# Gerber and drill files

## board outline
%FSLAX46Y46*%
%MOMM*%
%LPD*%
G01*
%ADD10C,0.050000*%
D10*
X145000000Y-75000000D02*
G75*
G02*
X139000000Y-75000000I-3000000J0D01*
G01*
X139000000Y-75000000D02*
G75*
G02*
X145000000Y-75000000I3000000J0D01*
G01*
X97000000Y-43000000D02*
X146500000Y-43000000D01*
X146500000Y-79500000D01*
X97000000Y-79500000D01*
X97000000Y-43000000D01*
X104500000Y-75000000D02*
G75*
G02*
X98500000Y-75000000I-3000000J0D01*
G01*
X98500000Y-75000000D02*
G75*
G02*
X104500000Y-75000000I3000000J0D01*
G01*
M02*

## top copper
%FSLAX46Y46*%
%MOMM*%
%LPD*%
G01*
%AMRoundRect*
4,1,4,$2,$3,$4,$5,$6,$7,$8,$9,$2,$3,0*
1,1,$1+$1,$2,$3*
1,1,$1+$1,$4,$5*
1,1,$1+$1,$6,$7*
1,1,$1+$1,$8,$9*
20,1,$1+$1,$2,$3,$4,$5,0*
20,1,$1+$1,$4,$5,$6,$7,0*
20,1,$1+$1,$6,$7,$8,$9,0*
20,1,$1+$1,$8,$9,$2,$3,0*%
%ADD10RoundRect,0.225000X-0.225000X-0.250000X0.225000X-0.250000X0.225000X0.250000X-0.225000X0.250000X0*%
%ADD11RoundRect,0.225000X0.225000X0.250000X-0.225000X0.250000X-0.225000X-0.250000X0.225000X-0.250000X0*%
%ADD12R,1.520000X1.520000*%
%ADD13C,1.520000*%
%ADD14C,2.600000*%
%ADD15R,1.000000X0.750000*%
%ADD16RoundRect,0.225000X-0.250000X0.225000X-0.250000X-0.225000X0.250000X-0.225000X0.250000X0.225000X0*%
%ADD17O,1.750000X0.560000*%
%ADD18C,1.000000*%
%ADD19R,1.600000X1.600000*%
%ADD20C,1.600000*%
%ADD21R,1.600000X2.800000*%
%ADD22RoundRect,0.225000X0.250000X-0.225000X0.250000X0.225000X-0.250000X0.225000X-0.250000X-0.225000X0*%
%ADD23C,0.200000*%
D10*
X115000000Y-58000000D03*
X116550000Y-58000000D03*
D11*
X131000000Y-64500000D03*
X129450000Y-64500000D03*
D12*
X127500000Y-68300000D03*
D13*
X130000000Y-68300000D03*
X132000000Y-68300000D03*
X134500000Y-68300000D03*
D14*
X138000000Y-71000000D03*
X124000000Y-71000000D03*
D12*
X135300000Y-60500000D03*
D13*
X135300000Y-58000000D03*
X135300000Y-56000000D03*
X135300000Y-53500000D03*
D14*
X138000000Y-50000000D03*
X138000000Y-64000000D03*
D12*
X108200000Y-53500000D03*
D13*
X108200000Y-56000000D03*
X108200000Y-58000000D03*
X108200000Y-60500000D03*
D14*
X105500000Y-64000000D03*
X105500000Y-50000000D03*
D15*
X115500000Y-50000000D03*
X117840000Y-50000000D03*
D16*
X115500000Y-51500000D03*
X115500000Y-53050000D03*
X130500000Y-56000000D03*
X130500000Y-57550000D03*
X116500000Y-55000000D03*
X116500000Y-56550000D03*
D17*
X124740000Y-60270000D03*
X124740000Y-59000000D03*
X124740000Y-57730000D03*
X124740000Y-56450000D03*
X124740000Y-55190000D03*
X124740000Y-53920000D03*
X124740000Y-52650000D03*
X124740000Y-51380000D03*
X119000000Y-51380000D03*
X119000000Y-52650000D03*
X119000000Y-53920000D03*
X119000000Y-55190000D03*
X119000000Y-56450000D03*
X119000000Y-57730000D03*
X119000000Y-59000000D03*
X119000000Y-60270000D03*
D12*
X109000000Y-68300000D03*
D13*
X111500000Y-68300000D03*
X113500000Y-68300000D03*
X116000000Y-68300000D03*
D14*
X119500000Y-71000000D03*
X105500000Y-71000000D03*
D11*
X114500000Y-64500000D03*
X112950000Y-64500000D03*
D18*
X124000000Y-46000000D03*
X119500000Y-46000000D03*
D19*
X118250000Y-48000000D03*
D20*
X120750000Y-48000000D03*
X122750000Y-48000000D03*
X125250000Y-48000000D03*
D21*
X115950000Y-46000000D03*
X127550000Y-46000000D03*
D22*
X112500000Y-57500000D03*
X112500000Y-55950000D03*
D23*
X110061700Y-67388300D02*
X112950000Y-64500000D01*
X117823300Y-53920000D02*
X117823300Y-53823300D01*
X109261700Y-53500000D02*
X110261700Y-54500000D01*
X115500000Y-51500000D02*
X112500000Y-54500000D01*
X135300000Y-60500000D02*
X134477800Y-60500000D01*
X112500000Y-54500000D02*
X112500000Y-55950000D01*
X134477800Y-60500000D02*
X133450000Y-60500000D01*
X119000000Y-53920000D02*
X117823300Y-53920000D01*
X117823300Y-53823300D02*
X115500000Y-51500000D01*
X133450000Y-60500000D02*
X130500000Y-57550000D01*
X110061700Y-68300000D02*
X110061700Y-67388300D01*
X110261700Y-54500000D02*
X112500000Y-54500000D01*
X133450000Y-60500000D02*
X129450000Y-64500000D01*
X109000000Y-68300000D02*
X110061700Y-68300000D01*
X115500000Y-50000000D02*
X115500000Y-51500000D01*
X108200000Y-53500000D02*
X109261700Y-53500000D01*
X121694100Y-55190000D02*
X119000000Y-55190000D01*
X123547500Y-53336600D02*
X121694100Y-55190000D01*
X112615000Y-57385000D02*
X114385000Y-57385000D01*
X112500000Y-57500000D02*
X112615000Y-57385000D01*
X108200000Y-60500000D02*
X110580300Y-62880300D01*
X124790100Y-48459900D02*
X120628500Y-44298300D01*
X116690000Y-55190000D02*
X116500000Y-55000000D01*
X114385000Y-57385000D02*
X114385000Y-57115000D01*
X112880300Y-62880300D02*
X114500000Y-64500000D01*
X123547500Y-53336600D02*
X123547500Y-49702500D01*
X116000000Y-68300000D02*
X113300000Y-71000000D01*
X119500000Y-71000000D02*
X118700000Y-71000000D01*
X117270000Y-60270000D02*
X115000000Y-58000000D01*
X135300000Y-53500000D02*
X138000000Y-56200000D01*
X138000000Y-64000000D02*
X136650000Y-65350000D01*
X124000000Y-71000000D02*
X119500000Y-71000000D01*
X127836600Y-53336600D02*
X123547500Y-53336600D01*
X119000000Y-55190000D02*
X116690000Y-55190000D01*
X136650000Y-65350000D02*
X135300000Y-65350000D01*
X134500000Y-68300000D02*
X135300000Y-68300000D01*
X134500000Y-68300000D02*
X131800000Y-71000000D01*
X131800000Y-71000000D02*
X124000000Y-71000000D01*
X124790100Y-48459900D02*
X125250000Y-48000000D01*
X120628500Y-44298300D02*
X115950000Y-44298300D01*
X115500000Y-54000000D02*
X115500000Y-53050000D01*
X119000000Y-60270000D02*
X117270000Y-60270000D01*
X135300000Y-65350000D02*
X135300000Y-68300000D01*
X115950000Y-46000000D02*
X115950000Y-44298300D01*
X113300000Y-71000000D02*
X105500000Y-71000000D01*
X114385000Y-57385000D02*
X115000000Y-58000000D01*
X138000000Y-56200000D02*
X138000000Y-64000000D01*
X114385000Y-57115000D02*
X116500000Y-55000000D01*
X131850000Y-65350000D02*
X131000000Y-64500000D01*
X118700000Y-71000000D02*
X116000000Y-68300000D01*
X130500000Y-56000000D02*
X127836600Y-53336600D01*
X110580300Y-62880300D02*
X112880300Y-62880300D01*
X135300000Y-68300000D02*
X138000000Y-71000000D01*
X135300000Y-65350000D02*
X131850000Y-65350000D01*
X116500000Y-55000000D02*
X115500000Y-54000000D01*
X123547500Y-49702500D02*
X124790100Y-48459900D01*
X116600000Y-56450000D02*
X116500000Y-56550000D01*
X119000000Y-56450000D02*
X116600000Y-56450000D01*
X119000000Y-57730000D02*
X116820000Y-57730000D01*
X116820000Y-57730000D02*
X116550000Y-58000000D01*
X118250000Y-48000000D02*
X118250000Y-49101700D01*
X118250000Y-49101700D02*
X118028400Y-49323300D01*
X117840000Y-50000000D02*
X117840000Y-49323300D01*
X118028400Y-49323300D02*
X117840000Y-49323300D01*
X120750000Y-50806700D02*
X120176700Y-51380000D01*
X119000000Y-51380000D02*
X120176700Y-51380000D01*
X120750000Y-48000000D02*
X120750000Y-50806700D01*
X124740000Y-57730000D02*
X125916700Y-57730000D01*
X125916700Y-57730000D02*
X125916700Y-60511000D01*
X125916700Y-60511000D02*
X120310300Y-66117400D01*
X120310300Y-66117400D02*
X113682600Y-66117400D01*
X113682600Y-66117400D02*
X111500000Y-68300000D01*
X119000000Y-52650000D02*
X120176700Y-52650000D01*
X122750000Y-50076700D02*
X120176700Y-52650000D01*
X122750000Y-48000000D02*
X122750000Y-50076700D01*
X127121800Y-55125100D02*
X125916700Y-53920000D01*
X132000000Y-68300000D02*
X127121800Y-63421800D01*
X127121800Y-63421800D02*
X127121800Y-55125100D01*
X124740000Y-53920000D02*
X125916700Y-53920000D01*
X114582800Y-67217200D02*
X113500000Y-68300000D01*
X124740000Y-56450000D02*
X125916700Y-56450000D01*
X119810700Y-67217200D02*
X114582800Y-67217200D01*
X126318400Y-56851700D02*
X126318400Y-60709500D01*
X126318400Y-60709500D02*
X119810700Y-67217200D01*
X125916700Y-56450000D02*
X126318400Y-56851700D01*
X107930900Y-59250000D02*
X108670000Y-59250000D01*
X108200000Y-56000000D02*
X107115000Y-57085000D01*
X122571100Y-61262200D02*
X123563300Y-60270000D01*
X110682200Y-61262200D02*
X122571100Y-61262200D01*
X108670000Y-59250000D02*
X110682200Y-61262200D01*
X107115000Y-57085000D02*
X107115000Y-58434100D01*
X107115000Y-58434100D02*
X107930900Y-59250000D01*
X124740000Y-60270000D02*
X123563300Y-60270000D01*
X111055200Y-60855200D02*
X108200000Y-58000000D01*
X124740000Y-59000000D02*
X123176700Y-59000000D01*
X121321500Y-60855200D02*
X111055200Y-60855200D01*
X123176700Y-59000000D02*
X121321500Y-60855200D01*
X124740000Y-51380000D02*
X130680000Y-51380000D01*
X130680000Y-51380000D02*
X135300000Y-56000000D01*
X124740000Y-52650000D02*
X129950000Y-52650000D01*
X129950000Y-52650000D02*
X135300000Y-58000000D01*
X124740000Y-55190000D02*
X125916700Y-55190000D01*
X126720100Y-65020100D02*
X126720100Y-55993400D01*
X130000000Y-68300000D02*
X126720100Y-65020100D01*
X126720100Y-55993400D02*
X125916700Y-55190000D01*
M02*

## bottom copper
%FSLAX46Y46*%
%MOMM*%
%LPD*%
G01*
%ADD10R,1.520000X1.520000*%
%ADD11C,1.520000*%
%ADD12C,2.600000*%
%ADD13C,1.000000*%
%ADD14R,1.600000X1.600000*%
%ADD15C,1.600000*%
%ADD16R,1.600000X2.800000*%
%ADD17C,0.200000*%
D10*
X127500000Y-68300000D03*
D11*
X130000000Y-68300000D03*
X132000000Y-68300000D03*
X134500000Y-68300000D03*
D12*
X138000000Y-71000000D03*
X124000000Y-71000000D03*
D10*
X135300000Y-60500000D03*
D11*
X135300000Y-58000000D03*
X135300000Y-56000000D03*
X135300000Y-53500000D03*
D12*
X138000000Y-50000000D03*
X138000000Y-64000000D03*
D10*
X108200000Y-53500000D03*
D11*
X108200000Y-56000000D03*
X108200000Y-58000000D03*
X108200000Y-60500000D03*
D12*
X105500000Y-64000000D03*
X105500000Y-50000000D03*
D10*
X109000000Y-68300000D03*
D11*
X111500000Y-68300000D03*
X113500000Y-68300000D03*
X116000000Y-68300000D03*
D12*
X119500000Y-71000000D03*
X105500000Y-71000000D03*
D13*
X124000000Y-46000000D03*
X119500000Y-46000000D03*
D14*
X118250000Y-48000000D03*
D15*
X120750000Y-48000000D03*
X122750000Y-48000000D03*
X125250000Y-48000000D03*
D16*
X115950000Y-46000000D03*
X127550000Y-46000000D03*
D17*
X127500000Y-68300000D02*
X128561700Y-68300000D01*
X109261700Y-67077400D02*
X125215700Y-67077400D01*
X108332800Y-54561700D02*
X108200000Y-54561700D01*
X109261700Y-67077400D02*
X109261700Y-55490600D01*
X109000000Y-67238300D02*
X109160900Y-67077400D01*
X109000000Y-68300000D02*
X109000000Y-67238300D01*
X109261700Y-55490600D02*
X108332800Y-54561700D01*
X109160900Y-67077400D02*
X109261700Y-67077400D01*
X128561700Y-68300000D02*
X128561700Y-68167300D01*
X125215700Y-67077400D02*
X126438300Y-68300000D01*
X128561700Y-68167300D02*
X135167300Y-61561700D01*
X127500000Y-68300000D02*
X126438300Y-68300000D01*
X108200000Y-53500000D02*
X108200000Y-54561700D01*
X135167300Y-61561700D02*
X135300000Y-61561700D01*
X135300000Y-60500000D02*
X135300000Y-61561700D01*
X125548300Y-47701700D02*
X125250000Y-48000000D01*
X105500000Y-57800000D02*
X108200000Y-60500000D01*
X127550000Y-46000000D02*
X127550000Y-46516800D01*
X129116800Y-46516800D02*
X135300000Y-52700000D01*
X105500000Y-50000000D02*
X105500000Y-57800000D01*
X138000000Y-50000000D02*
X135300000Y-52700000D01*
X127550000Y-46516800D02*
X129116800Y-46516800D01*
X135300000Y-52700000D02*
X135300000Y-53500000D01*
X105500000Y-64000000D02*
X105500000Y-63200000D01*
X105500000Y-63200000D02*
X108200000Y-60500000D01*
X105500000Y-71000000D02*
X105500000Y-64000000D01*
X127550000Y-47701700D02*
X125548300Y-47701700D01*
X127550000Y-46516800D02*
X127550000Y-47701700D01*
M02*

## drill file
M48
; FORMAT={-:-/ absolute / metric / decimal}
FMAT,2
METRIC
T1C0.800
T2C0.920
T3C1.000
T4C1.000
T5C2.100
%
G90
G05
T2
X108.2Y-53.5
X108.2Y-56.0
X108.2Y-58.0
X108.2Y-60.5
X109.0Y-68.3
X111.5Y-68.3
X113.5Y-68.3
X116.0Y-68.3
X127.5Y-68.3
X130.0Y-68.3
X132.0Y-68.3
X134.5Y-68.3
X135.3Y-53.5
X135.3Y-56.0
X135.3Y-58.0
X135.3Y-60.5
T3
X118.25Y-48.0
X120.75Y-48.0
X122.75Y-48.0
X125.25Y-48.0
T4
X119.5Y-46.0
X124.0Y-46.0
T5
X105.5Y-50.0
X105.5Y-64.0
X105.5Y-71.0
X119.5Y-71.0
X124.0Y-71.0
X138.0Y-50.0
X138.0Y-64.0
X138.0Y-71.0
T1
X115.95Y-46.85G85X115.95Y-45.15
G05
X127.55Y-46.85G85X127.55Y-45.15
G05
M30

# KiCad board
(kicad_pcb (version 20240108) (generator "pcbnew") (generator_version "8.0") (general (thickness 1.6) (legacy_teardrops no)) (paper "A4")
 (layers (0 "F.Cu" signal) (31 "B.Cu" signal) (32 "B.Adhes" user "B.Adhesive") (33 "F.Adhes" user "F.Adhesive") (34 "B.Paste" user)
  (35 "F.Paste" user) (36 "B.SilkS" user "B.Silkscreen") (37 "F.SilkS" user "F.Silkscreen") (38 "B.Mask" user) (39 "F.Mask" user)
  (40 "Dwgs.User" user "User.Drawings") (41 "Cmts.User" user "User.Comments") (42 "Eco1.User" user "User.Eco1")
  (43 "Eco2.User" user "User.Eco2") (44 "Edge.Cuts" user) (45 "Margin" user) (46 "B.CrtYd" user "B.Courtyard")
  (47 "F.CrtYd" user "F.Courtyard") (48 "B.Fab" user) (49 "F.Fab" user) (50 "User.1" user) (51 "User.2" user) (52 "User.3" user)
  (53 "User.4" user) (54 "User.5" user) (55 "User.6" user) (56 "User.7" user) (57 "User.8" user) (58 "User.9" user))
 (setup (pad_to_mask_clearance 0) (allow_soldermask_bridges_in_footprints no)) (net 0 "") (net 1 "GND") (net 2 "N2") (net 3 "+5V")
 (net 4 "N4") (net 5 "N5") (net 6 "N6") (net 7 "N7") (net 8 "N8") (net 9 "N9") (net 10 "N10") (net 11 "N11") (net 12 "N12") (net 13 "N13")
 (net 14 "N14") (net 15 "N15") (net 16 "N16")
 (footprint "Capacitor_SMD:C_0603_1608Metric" (layer "F.Cu") (at 115.775 58)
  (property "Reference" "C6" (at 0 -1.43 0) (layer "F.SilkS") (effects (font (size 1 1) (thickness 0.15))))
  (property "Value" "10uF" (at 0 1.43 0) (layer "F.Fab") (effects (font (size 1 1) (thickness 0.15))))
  (pad "1" smd roundrect (at -0.775 0) (size 0.9 0.95) (layers "F.Cu" "F.Paste" "F.Mask") (roundrect_rratio 0.25) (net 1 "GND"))
  (pad "2" smd roundrect (at 0.775 0) (size 0.9 0.95) (layers "F.Cu" "F.Paste" "F.Mask") (roundrect_rratio 0.25) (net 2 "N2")))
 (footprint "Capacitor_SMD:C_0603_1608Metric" (layer "F.Cu") (at 130.225 64.5 180)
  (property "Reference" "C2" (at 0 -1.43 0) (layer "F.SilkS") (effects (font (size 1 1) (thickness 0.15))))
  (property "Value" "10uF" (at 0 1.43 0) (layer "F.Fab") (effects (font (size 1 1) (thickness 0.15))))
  (pad "1" smd roundrect (at -0.775 0 180) (size 0.9 0.95) (layers "F.Cu" "F.Paste" "F.Mask") (roundrect_rratio 0.25) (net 1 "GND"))
  (pad "2" smd roundrect (at 0.775 0 180) (size 0.9 0.95) (layers "F.Cu" "F.Paste" "F.Mask") (roundrect_rratio 0.25) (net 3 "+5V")))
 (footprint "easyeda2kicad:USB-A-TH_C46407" (layer "F.Cu") (at 131 69.65)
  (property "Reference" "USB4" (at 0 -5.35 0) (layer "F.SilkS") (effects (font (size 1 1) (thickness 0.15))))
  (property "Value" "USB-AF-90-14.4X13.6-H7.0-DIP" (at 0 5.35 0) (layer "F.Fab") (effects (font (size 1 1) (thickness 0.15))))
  (pad "1" thru_hole rect (at -3.5 -1.35) (size 1.52 1.52) (drill 0.919988) (layers "*.Cu" "*.Mask") (remove_unused_layers no) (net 3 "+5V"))
  (pad "2" thru_hole circle (at -1 -1.35) (size 1.52 1.52) (drill 0.919988) (layers "*.Cu" "*.Mask") (remove_unused_layers no) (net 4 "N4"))
  (pad "3" thru_hole circle (at 1 -1.35) (size 1.52 1.52) (drill 0.919988) (layers "*.Cu" "*.Mask") (remove_unused_layers no) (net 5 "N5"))
  (pad "4" thru_hole circle (at 3.5 -1.35) (size 1.52 1.52) (drill 0.919988) (layers "*.Cu" "*.Mask") (remove_unused_layers no)
   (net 1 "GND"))
  (pad "5" thru_hole circle (at 7 1.35) (size 2.6 2.6) (drill 2.100021) (layers "*.Cu" "*.Mask") (remove_unused_layers no) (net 1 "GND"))
  (pad "6" thru_hole circle (at -7 1.35) (size 2.6 2.6) (drill 2.100021) (layers "*.Cu" "*.Mask") (remove_unused_layers no) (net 1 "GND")))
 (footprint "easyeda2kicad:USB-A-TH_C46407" (layer "F.Cu") (at 136.65 57 90)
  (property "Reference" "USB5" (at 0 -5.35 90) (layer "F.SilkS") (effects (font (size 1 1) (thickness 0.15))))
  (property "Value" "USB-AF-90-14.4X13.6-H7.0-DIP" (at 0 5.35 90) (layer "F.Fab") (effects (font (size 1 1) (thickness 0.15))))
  (pad "1" thru_hole rect (at -3.5 -1.35 90) (size 1.52 1.52) (drill 0.919988) (layers "*.Cu" "*.Mask") (remove_unused_layers no)
   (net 3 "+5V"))
  (pad "2" thru_hole circle (at -1 -1.35 90) (size 1.52 1.52) (drill 0.919988) (layers "*.Cu" "*.Mask") (remove_unused_layers no)
   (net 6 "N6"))
  (pad "3" thru_hole circle (at 1 -1.35 90) (size 1.52 1.52) (drill 0.919988) (layers "*.Cu" "*.Mask") (remove_unused_layers no)
   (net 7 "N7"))
  (pad "4" thru_hole circle (at 3.5 -1.35 90) (size 1.52 1.52) (drill 0.919988) (layers "*.Cu" "*.Mask") (remove_unused_layers no)
   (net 1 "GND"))
  (pad "5" thru_hole circle (at 7 1.35 90) (size 2.6 2.6) (drill 2.100021) (layers "*.Cu" "*.Mask") (remove_unused_layers no) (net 1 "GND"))
  (pad "6" thru_hole circle (at -7 1.35 90) (size 2.6 2.6) (drill 2.100021) (layers "*.Cu" "*.Mask") (remove_unused_layers no) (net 1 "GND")))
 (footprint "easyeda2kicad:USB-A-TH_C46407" (layer "F.Cu") (at 106.85 57 -90)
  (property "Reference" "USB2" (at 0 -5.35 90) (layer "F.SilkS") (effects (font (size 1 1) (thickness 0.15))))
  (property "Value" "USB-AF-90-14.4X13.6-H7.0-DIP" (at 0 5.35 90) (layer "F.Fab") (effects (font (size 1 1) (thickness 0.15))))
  (pad "1" thru_hole rect (at -3.5 -1.35 270) (size 1.52 1.52) (drill 0.919988) (layers "*.Cu" "*.Mask") (remove_unused_layers no)
   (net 3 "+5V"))
  (pad "2" thru_hole circle (at -1 -1.35 270) (size 1.52 1.52) (drill 0.919988) (layers "*.Cu" "*.Mask") (remove_unused_layers no)
   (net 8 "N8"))
  (pad "3" thru_hole circle (at 1 -1.35 270) (size 1.52 1.52) (drill 0.919988) (layers "*.Cu" "*.Mask") (remove_unused_layers no)
   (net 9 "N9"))
  (pad "4" thru_hole circle (at 3.5 -1.35 270) (size 1.52 1.52) (drill 0.919988) (layers "*.Cu" "*.Mask") (remove_unused_layers no)
   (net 1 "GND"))
  (pad "5" thru_hole circle (at 7 1.35 270) (size 2.6 2.6) (drill 2.100021) (layers "*.Cu" "*.Mask") (remove_unused_layers no) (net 1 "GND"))
  (pad "6" thru_hole circle (at -7 1.35 270) (size 2.6 2.6) (drill 2.100021) (layers "*.Cu" "*.Mask") (remove_unused_layers no)
   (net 1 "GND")))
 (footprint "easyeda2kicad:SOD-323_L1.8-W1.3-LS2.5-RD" (layer "F.Cu") (at 116.67 50)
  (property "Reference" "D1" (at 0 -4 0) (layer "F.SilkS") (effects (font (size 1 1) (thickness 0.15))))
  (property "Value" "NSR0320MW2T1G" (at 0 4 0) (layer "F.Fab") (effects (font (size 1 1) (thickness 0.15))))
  (pad "1" smd rect (at -1.17 0) (size 1 0.75) (layers "F.Cu" "F.Paste" "F.Mask") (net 3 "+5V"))
  (pad "2" smd rect (at 1.17 0) (size 1 0.75) (layers "F.Cu" "F.Paste" "F.Mask") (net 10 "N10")))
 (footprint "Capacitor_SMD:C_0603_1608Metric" (layer "F.Cu") (at 115.5 52.275 -90)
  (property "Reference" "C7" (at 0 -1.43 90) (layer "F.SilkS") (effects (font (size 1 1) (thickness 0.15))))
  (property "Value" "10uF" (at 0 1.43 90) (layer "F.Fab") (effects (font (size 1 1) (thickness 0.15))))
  (pad "1" smd roundrect (at -0.775 0 270) (size 0.9 0.95) (layers "F.Cu" "F.Paste" "F.Mask") (roundrect_rratio 0.25) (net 3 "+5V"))
  (pad "2" smd roundrect (at 0.775 0 270) (size 0.9 0.95) (layers "F.Cu" "F.Paste" "F.Mask") (roundrect_rratio 0.25) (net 1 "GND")))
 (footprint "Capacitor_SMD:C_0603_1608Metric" (layer "F.Cu") (at 130.5 56.775 -90)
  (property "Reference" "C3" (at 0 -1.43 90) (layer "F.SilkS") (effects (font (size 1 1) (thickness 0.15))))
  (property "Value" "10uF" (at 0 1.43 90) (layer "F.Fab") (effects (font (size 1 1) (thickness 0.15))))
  (pad "1" smd roundrect (at -0.775 0 270) (size 0.9 0.95) (layers "F.Cu" "F.Paste" "F.Mask") (roundrect_rratio 0.25) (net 1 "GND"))
  (pad "2" smd roundrect (at 0.775 0 270) (size 0.9 0.95) (layers "F.Cu" "F.Paste" "F.Mask") (roundrect_rratio 0.25) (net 3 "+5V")))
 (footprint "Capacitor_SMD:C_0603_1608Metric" (layer "F.Cu") (at 116.5 55.775 -90)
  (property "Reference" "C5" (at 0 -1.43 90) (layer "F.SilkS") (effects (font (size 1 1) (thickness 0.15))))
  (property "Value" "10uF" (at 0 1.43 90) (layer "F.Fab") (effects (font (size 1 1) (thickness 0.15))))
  (pad "1" smd roundrect (at -0.775 0 270) (size 0.9 0.95) (layers "F.Cu" "F.Paste" "F.Mask") (roundrect_rratio 0.25) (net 1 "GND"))
  (pad "2" smd roundrect (at 0.775 0 270) (size 0.9 0.95) (layers "F.Cu" "F.Paste" "F.Mask") (roundrect_rratio 0.25) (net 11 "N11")))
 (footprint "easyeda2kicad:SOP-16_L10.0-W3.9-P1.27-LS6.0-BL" (layer "F.Cu") (at 121.87 55.82 90)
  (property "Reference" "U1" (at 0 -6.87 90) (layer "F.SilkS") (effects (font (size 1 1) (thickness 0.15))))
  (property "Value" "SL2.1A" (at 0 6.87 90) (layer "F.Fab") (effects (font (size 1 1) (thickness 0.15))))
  (pad "1" smd oval (at -4.45 2.87 90) (size 0.56 1.75) (layers "F.Cu" "F.Paste" "F.Mask") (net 8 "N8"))
  (pad "2" smd oval (at -3.18 2.87 90) (size 0.56 1.75) (layers "F.Cu" "F.Paste" "F.Mask") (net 9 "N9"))
  (pad "3" smd oval (at -1.91 2.87 90) (size 0.56 1.75) (layers "F.Cu" "F.Paste" "F.Mask") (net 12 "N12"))
  (pad "4" smd oval (at -0.63 2.87 90) (size 0.56 1.75) (layers "F.Cu" "F.Paste" "F.Mask") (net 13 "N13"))
  (pad "5" smd oval (at 0.63 2.87 90) (size 0.56 1.75) (layers "F.Cu" "F.Paste" "F.Mask") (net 4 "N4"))
  (pad "6" smd oval (at 1.9 2.87 90) (size 0.56 1.75) (layers "F.Cu" "F.Paste" "F.Mask") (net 5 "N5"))
  (pad "7" smd oval (at 3.17 2.87 90) (size 0.56 1.75) (layers "F.Cu" "F.Paste" "F.Mask") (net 6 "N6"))
  (pad "8" smd oval (at 4.44 2.87 90) (size 0.56 1.75) (layers "F.Cu" "F.Paste" "F.Mask") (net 7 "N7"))
  (pad "9" smd oval (at 4.44 -2.87 90) (size 0.56 1.75) (layers "F.Cu" "F.Paste" "F.Mask") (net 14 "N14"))
  (pad "10" smd oval (at 3.17 -2.87 90) (size 0.56 1.75) (layers "F.Cu" "F.Paste" "F.Mask") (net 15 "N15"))
  (pad "11" smd oval (at 1.9 -2.87 90) (size 0.56 1.75) (layers "F.Cu" "F.Paste" "F.Mask") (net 3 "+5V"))
  (pad "12" smd oval (at 0.63 -2.87 90) (size 0.56 1.75) (layers "F.Cu" "F.Paste" "F.Mask") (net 1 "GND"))
  (pad "13" smd oval (at -0.63 -2.87 90) (size 0.56 1.75) (layers "F.Cu" "F.Paste" "F.Mask") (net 11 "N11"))
  (pad "14" smd oval (at -1.91 -2.87 90) (size 0.56 1.75) (layers "F.Cu" "F.Paste" "F.Mask") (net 2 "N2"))
  (pad "15" smd oval (at -3.18 -2.87 90) (size 0.56 1.75) (layers "F.Cu" "F.Paste" "F.Mask") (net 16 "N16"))
  (pad "16" smd oval (at -4.45 -2.87 90) (size 0.56 1.75) (layers "F.Cu" "F.Paste" "F.Mask") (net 1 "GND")))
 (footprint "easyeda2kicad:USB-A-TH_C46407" (layer "F.Cu") (at 112.5 69.65)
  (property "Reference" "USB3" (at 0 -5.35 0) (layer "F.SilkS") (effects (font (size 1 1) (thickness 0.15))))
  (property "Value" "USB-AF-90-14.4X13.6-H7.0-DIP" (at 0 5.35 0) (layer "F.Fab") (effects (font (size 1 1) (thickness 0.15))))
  (pad "1" thru_hole rect (at -3.5 -1.35) (size 1.52 1.52) (drill 0.919988) (layers "*.Cu" "*.Mask") (remove_unused_layers no) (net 3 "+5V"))
  (pad "2" thru_hole circle (at -1 -1.35) (size 1.52 1.52) (drill 0.919988) (layers "*.Cu" "*.Mask") (remove_unused_layers no)
   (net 12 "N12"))
  (pad "3" thru_hole circle (at 1 -1.35) (size 1.52 1.52) (drill 0.919988) (layers "*.Cu" "*.Mask") (remove_unused_layers no) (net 13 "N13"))
  (pad "4" thru_hole circle (at 3.5 -1.35) (size 1.52 1.52) (drill 0.919988) (layers "*.Cu" "*.Mask") (remove_unused_layers no)
   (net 1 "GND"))
  (pad "5" thru_hole circle (at 7 1.35) (size 2.6 2.6) (drill 2.100021) (layers "*.Cu" "*.Mask") (remove_unused_layers no) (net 1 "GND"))
  (pad "6" thru_hole circle (at -7 1.35) (size 2.6 2.6) (drill 2.100021) (layers "*.Cu" "*.Mask") (remove_unused_layers no) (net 1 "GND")))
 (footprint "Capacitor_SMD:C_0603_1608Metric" (layer "F.Cu") (at 113.725 64.5 180)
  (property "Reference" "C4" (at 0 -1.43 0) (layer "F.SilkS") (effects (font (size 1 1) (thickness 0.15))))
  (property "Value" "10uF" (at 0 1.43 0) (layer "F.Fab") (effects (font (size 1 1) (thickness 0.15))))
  (pad "1" smd roundrect (at -0.775 0 180) (size 0.9 0.95) (layers "F.Cu" "F.Paste" "F.Mask") (roundrect_rratio 0.25) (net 1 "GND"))
  (pad "2" smd roundrect (at 0.775 0 180) (size 0.9 0.95) (layers "F.Cu" "F.Paste" "F.Mask") (roundrect_rratio 0.25) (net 3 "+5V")))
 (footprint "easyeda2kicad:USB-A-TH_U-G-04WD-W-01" (layer "F.Cu") (at 121.75 47 180)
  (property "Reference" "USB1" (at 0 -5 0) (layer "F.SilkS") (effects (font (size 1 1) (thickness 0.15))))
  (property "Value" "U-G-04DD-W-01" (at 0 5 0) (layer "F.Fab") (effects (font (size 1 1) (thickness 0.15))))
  (pad "" thru_hole circle (at -2.25 1 180) (size 1 1) (drill 1) (layers "*.Cu" "*.Mask") (remove_unused_layers no))
  (pad "" thru_hole circle (at 2.25 1 180) (size 1 1) (drill 1) (layers "*.Cu" "*.Mask") (remove_unused_layers no))
  (pad "1" thru_hole rect (at 3.5 -1 180) (size 1.6 1.6) (drill 0.999998) (layers "*.Cu" "*.Mask") (remove_unused_layers no) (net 10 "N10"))
  (pad "2" thru_hole circle (at 1 -1 180) (size 1.6 1.6) (drill 0.999998) (layers "*.Cu" "*.Mask") (remove_unused_layers no) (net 14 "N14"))
  (pad "3" thru_hole circle (at -1 -1 180) (size 1.6 1.6) (drill 0.999998) (layers "*.Cu" "*.Mask") (remove_unused_layers no) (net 15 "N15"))
  (pad "4" thru_hole circle (at -3.5 -1 180) (size 1.6 1.6) (drill 0.999998) (layers "*.Cu" "*.Mask") (remove_unused_layers no)
   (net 1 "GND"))
  (pad "5" thru_hole rect (at 5.8 1 180) (size 1.6 2.8) (drill oval 0.799998 2.499995) (layers "*.Cu" "*.Mask") (remove_unused_layers no)
   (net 1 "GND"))
  (pad "6" thru_hole rect (at -5.8 1 180) (size 1.6 2.8) (drill oval 0.799998 2.499995) (layers "*.Cu" "*.Mask") (remove_unused_layers no)
   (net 1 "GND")))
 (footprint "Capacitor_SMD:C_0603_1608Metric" (layer "F.Cu") (at 112.5 56.725 90)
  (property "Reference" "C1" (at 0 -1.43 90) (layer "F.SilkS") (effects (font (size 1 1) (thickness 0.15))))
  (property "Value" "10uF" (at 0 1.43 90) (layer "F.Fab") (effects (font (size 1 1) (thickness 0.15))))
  (pad "1" smd roundrect (at -0.775 0 90) (size 0.9 0.95) (layers "F.Cu" "F.Paste" "F.Mask") (roundrect_rratio 0.25) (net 1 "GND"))
  (pad "2" smd roundrect (at 0.775 0 90) (size 0.9 0.95) (layers "F.Cu" "F.Paste" "F.Mask") (roundrect_rratio 0.25) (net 3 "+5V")))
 (gr_circle (center 142 75) (end 145 75) (stroke (width 0.05) (type default)) (fill none) (layer "Edge.Cuts"))
 (gr_rect (start 97 43) (end 146.5 79.5) (stroke (width 0.05) (type default)) (fill none) (layer "Edge.Cuts"))
 (gr_circle (center 101.5 75) (end 104.5 75) (stroke (width 0.05) (type default)) (fill none) (layer "Edge.Cuts"))
 (segment (start 110.0617 67.3883) (end 112.95 64.5) (width 0.2) (layer "F.Cu") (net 3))
 (segment (start 117.8233 53.92) (end 117.8233 53.8233) (width 0.2) (layer "F.Cu") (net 3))
 (segment (start 109.2617 53.5) (end 110.2617 54.5) (width 0.2) (layer "F.Cu") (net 3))
 (segment (start 115.5 51.5) (end 112.5 54.5) (width 0.2) (layer "F.Cu") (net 3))
 (segment (start 135.3 60.5) (end 134.4778 60.5) (width 0.2) (layer "F.Cu") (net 3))
 (segment (start 112.5 54.5) (end 112.5 55.95) (width 0.2) (layer "F.Cu") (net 3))
 (segment (start 134.4778 60.5) (end 133.45 60.5) (width 0.2) (layer "F.Cu") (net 3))
 (segment (start 119 53.92) (end 117.8233 53.92) (width 0.2) (layer "F.Cu") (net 3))
 (segment (start 117.8233 53.8233) (end 115.5 51.5) (width 0.2) (layer "F.Cu") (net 3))
 (segment (start 133.45 60.5) (end 130.5 57.55) (width 0.2) (layer "F.Cu") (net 3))
 (segment (start 110.0617 68.3) (end 110.0617 67.3883) (width 0.2) (layer "F.Cu") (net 3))
 (segment (start 110.2617 54.5) (end 112.5 54.5) (width 0.2) (layer "F.Cu") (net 3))
 (segment (start 133.45 60.5) (end 129.45 64.5) (width 0.2) (layer "F.Cu") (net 3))
 (segment (start 109 68.3) (end 110.0617 68.3) (width 0.2) (layer "F.Cu") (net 3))
 (segment (start 115.5 50) (end 115.5 51.5) (width 0.2) (layer "F.Cu") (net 3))
 (segment (start 108.2 53.5) (end 109.2617 53.5) (width 0.2) (layer "F.Cu") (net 3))
 (segment (start 127.5 68.3) (end 128.5617 68.3) (width 0.2) (layer "B.Cu") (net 3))
 (segment (start 109.2617 67.0774) (end 125.2157 67.0774) (width 0.2) (layer "B.Cu") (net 3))
 (segment (start 108.3328 54.5617) (end 108.2 54.5617) (width 0.2) (layer "B.Cu") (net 3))
 (segment (start 109.2617 67.0774) (end 109.2617 55.4906) (width 0.2) (layer "B.Cu") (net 3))
 (segment (start 109 67.2383) (end 109.1609 67.0774) (width 0.2) (layer "B.Cu") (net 3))
 (segment (start 109 68.3) (end 109 67.2383) (width 0.2) (layer "B.Cu") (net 3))
 (segment (start 109.2617 55.4906) (end 108.3328 54.5617) (width 0.2) (layer "B.Cu") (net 3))
 (segment (start 109.1609 67.0774) (end 109.2617 67.0774) (width 0.2) (layer "B.Cu") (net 3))
 (segment (start 128.5617 68.3) (end 128.5617 68.1673) (width 0.2) (layer "B.Cu") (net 3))
 (segment (start 125.2157 67.0774) (end 126.4383 68.3) (width 0.2) (layer "B.Cu") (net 3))
 (segment (start 128.5617 68.1673) (end 135.1673 61.5617) (width 0.2) (layer "B.Cu") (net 3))
 (segment (start 127.5 68.3) (end 126.4383 68.3) (width 0.2) (layer "B.Cu") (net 3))
 (segment (start 108.2 53.5) (end 108.2 54.5617) (width 0.2) (layer "B.Cu") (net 3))
 (segment (start 135.1673 61.5617) (end 135.3 61.5617) (width 0.2) (layer "B.Cu") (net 3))
 (segment (start 135.3 60.5) (end 135.3 61.5617) (width 0.2) (layer "B.Cu") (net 3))
 (segment (start 121.6941 55.19) (end 119 55.19) (width 0.2) (layer "F.Cu") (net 1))
 (segment (start 123.5475 53.3366) (end 121.6941 55.19) (width 0.2) (layer "F.Cu") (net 1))
 (segment (start 112.615 57.385) (end 114.385 57.385) (width 0.2) (layer "F.Cu") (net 1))
 (segment (start 112.5 57.5) (end 112.615 57.385) (width 0.2) (layer "F.Cu") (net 1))
 (segment (start 108.2 60.5) (end 110.5803 62.8803) (width 0.2) (layer "F.Cu") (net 1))
 (segment (start 124.7901 48.4599) (end 120.6285 44.2983) (width 0.2) (layer "F.Cu") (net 1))
 (segment (start 116.69 55.19) (end 116.5 55) (width 0.2) (layer "F.Cu") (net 1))
 (segment (start 114.385 57.385) (end 114.385 57.115) (width 0.2) (layer "F.Cu") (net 1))
 (segment (start 112.8803 62.8803) (end 114.5 64.5) (width 0.2) (layer "F.Cu") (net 1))
 (segment (start 123.5475 53.3366) (end 123.5475 49.7025) (width 0.2) (layer "F.Cu") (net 1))
 (segment (start 116 68.3) (end 113.3 71) (width 0.2) (layer "F.Cu") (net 1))
 (segment (start 119.5 71) (end 118.7 71) (width 0.2) (layer "F.Cu") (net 1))
 (segment (start 117.27 60.27) (end 115 58) (width 0.2) (layer "F.Cu") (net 1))
 (segment (start 135.3 53.5) (end 138 56.2) (width 0.2) (layer "F.Cu") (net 1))
 (segment (start 138 64) (end 136.65 65.35) (width 0.2) (layer "F.Cu") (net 1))
 (segment (start 124 71) (end 119.5 71) (width 0.2) (layer "F.Cu") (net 1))
 (segment (start 127.8366 53.3366) (end 123.5475 53.3366) (width 0.2) (layer "F.Cu") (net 1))
 (segment (start 119 55.19) (end 116.69 55.19) (width 0.2) (layer "F.Cu") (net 1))
 (segment (start 136.65 65.35) (end 135.3 65.35) (width 0.2) (layer "F.Cu") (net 1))
 (segment (start 134.5 68.3) (end 135.3 68.3) (width 0.2) (layer "F.Cu") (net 1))
 (segment (start 134.5 68.3) (end 131.8 71) (width 0.2) (layer "F.Cu") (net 1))
 (segment (start 131.8 71) (end 124 71) (width 0.2) (layer "F.Cu") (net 1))
 (segment (start 124.7901 48.4599) (end 125.25 48) (width 0.2) (layer "F.Cu") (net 1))
 (segment (start 120.6285 44.2983) (end 115.95 44.2983) (width 0.2) (layer "F.Cu") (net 1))
 (segment (start 115.5 54) (end 115.5 53.05) (width 0.2) (layer "F.Cu") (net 1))
 (segment (start 119 60.27) (end 117.27 60.27) (width 0.2) (layer "F.Cu") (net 1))
 (segment (start 135.3 65.35) (end 135.3 68.3) (width 0.2) (layer "F.Cu") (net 1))
 (segment (start 115.95 46) (end 115.95 44.2983) (width 0.2) (layer "F.Cu") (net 1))
 (segment (start 113.3 71) (end 105.5 71) (width 0.2) (layer "F.Cu") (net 1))
 (segment (start 114.385 57.385) (end 115 58) (width 0.2) (layer "F.Cu") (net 1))
 (segment (start 138 56.2) (end 138 64) (width 0.2) (layer "F.Cu") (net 1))
 (segment (start 114.385 57.115) (end 116.5 55) (width 0.2) (layer "F.Cu") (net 1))
 (segment (start 131.85 65.35) (end 131 64.5) (width 0.2) (layer "F.Cu") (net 1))
 (segment (start 118.7 71) (end 116 68.3) (width 0.2) (layer "F.Cu") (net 1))
 (segment (start 130.5 56) (end 127.8366 53.3366) (width 0.2) (layer "F.Cu") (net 1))
 (segment (start 110.5803 62.8803) (end 112.8803 62.8803) (width 0.2) (layer "F.Cu") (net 1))
 (segment (start 135.3 68.3) (end 138 71) (width 0.2) (layer "F.Cu") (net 1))
 (segment (start 135.3 65.35) (end 131.85 65.35) (width 0.2) (layer "F.Cu") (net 1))
 (segment (start 116.5 55) (end 115.5 54) (width 0.2) (layer "F.Cu") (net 1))
 (segment (start 123.5475 49.7025) (end 124.7901 48.4599) (width 0.2) (layer "F.Cu") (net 1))
 (segment (start 125.5483 47.7017) (end 125.25 48) (width 0.2) (layer "B.Cu") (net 1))
 (segment (start 105.5 57.8) (end 108.2 60.5) (width 0.2) (layer "B.Cu") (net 1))
 (segment (start 127.55 46) (end 127.55 46.5168) (width 0.2) (layer "B.Cu") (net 1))
 (segment (start 129.1168 46.5168) (end 135.3 52.7) (width 0.2) (layer "B.Cu") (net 1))
 (segment (start 105.5 50) (end 105.5 57.8) (width 0.2) (layer "B.Cu") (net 1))
 (segment (start 138 50) (end 135.3 52.7) (width 0.2) (layer "B.Cu") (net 1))
 (segment (start 127.55 46.5168) (end 129.1168 46.5168) (width 0.2) (layer "B.Cu") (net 1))
 (segment (start 135.3 52.7) (end 135.3 53.5) (width 0.2) (layer "B.Cu") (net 1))
 (segment (start 105.5 64) (end 105.5 63.2) (width 0.2) (layer "B.Cu") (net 1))
 (segment (start 105.5 63.2) (end 108.2 60.5) (width 0.2) (layer "B.Cu") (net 1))
 (segment (start 105.5 71) (end 105.5 64) (width 0.2) (layer "B.Cu") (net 1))
 (segment (start 127.55 47.7017) (end 125.5483 47.7017) (width 0.2) (layer "B.Cu") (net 1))
 (segment (start 127.55 46.5168) (end 127.55 47.7017) (width 0.2) (layer "B.Cu") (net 1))
 (segment (start 116.6 56.45) (end 116.5 56.55) (width 0.2) (layer "F.Cu") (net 11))
 (segment (start 119 56.45) (end 116.6 56.45) (width 0.2) (layer "F.Cu") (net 11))
 (segment (start 119 57.73) (end 116.82 57.73) (width 0.2) (layer "F.Cu") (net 2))
 (segment (start 116.82 57.73) (end 116.55 58) (width 0.2) (layer "F.Cu") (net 2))
 (segment (start 118.25 48) (end 118.25 49.1017) (width 0.2) (layer "F.Cu") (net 10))
 (segment (start 118.25 49.1017) (end 118.0284 49.3233) (width 0.2) (layer "F.Cu") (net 10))
 (segment (start 117.84 50) (end 117.84 49.3233) (width 0.2) (layer "F.Cu") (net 10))
 (segment (start 118.0284 49.3233) (end 117.84 49.3233) (width 0.2) (layer "F.Cu") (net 10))
 (segment (start 120.75 50.8067) (end 120.1767 51.38) (width 0.2) (layer "F.Cu") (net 14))
 (segment (start 119 51.38) (end 120.1767 51.38) (width 0.2) (layer "F.Cu") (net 14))
 (segment (start 120.75 48) (end 120.75 50.8067) (width 0.2) (layer "F.Cu") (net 14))
 (segment (start 124.74 57.73) (end 125.9167 57.73) (width 0.2) (layer "F.Cu") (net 12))
 (segment (start 125.9167 57.73) (end 125.9167 60.511) (width 0.2) (layer "F.Cu") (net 12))
 (segment (start 125.9167 60.511) (end 120.3103 66.1174) (width 0.2) (layer "F.Cu") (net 12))
 (segment (start 120.3103 66.1174) (end 113.6826 66.1174) (width 0.2) (layer "F.Cu") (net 12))
 (segment (start 113.6826 66.1174) (end 111.5 68.3) (width 0.2) (layer "F.Cu") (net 12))
 (segment (start 119 52.65) (end 120.1767 52.65) (width 0.2) (layer "F.Cu") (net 15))
 (segment (start 122.75 50.0767) (end 120.1767 52.65) (width 0.2) (layer "F.Cu") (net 15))
 (segment (start 122.75 48) (end 122.75 50.0767) (width 0.2) (layer "F.Cu") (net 15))
 (segment (start 127.1218 55.1251) (end 125.9167 53.92) (width 0.2) (layer "F.Cu") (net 5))
 (segment (start 132 68.3) (end 127.1218 63.4218) (width 0.2) (layer "F.Cu") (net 5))
 (segment (start 127.1218 63.4218) (end 127.1218 55.1251) (width 0.2) (layer "F.Cu") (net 5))
 (segment (start 124.74 53.92) (end 125.9167 53.92) (width 0.2) (layer "F.Cu") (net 5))
 (segment (start 114.5828 67.2172) (end 113.5 68.3) (width 0.2) (layer "F.Cu") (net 13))
 (segment (start 124.74 56.45) (end 125.9167 56.45) (width 0.2) (layer "F.Cu") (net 13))
 (segment (start 119.8107 67.2172) (end 114.5828 67.2172) (width 0.2) (layer "F.Cu") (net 13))
 (segment (start 126.3184 56.8517) (end 126.3184 60.7095) (width 0.2) (layer "F.Cu") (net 13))
 (segment (start 126.3184 60.7095) (end 119.8107 67.2172) (width 0.2) (layer "F.Cu") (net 13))
 (segment (start 125.9167 56.45) (end 126.3184 56.8517) (width 0.2) (layer "F.Cu") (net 13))
 (segment (start 107.9309 59.25) (end 108.67 59.25) (width 0.2) (layer "F.Cu") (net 8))
 (segment (start 108.2 56) (end 107.115 57.085) (width 0.2) (layer "F.Cu") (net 8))
 (segment (start 122.5711 61.2622) (end 123.5633 60.27) (width 0.2) (layer "F.Cu") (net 8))
 (segment (start 110.6822 61.2622) (end 122.5711 61.2622) (width 0.2) (layer "F.Cu") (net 8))
 (segment (start 108.67 59.25) (end 110.6822 61.2622) (width 0.2) (layer "F.Cu") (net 8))
 (segment (start 107.115 57.085) (end 107.115 58.4341) (width 0.2) (layer "F.Cu") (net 8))
 (segment (start 107.115 58.4341) (end 107.9309 59.25) (width 0.2) (layer "F.Cu") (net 8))
 (segment (start 124.74 60.27) (end 123.5633 60.27) (width 0.2) (layer "F.Cu") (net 8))
 (segment (start 111.0552 60.8552) (end 108.2 58) (width 0.2) (layer "F.Cu") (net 9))
 (segment (start 124.74 59) (end 123.1767 59) (width 0.2) (layer "F.Cu") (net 9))
 (segment (start 121.3215 60.8552) (end 111.0552 60.8552) (width 0.2) (layer "F.Cu") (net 9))
 (segment (start 123.1767 59) (end 121.3215 60.8552) (width 0.2) (layer "F.Cu") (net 9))
 (segment (start 124.74 51.38) (end 130.68 51.38) (width 0.2) (layer "F.Cu") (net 7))
 (segment (start 130.68 51.38) (end 135.3 56) (width 0.2) (layer "F.Cu") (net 7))
 (segment (start 124.74 52.65) (end 129.95 52.65) (width 0.2) (layer "F.Cu") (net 6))
 (segment (start 129.95 52.65) (end 135.3 58) (width 0.2) (layer "F.Cu") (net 6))
 (segment (start 124.74 55.19) (end 125.9167 55.19) (width 0.2) (layer "F.Cu") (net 4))
 (segment (start 126.7201 65.0201) (end 126.7201 55.9934) (width 0.2) (layer "F.Cu") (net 4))
 (segment (start 130 68.3) (end 126.7201 65.0201) (width 0.2) (layer "F.Cu") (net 4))
 (segment (start 126.7201 55.9934) (end 125.9167 55.19) (width 0.2) (layer "F.Cu") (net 4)))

